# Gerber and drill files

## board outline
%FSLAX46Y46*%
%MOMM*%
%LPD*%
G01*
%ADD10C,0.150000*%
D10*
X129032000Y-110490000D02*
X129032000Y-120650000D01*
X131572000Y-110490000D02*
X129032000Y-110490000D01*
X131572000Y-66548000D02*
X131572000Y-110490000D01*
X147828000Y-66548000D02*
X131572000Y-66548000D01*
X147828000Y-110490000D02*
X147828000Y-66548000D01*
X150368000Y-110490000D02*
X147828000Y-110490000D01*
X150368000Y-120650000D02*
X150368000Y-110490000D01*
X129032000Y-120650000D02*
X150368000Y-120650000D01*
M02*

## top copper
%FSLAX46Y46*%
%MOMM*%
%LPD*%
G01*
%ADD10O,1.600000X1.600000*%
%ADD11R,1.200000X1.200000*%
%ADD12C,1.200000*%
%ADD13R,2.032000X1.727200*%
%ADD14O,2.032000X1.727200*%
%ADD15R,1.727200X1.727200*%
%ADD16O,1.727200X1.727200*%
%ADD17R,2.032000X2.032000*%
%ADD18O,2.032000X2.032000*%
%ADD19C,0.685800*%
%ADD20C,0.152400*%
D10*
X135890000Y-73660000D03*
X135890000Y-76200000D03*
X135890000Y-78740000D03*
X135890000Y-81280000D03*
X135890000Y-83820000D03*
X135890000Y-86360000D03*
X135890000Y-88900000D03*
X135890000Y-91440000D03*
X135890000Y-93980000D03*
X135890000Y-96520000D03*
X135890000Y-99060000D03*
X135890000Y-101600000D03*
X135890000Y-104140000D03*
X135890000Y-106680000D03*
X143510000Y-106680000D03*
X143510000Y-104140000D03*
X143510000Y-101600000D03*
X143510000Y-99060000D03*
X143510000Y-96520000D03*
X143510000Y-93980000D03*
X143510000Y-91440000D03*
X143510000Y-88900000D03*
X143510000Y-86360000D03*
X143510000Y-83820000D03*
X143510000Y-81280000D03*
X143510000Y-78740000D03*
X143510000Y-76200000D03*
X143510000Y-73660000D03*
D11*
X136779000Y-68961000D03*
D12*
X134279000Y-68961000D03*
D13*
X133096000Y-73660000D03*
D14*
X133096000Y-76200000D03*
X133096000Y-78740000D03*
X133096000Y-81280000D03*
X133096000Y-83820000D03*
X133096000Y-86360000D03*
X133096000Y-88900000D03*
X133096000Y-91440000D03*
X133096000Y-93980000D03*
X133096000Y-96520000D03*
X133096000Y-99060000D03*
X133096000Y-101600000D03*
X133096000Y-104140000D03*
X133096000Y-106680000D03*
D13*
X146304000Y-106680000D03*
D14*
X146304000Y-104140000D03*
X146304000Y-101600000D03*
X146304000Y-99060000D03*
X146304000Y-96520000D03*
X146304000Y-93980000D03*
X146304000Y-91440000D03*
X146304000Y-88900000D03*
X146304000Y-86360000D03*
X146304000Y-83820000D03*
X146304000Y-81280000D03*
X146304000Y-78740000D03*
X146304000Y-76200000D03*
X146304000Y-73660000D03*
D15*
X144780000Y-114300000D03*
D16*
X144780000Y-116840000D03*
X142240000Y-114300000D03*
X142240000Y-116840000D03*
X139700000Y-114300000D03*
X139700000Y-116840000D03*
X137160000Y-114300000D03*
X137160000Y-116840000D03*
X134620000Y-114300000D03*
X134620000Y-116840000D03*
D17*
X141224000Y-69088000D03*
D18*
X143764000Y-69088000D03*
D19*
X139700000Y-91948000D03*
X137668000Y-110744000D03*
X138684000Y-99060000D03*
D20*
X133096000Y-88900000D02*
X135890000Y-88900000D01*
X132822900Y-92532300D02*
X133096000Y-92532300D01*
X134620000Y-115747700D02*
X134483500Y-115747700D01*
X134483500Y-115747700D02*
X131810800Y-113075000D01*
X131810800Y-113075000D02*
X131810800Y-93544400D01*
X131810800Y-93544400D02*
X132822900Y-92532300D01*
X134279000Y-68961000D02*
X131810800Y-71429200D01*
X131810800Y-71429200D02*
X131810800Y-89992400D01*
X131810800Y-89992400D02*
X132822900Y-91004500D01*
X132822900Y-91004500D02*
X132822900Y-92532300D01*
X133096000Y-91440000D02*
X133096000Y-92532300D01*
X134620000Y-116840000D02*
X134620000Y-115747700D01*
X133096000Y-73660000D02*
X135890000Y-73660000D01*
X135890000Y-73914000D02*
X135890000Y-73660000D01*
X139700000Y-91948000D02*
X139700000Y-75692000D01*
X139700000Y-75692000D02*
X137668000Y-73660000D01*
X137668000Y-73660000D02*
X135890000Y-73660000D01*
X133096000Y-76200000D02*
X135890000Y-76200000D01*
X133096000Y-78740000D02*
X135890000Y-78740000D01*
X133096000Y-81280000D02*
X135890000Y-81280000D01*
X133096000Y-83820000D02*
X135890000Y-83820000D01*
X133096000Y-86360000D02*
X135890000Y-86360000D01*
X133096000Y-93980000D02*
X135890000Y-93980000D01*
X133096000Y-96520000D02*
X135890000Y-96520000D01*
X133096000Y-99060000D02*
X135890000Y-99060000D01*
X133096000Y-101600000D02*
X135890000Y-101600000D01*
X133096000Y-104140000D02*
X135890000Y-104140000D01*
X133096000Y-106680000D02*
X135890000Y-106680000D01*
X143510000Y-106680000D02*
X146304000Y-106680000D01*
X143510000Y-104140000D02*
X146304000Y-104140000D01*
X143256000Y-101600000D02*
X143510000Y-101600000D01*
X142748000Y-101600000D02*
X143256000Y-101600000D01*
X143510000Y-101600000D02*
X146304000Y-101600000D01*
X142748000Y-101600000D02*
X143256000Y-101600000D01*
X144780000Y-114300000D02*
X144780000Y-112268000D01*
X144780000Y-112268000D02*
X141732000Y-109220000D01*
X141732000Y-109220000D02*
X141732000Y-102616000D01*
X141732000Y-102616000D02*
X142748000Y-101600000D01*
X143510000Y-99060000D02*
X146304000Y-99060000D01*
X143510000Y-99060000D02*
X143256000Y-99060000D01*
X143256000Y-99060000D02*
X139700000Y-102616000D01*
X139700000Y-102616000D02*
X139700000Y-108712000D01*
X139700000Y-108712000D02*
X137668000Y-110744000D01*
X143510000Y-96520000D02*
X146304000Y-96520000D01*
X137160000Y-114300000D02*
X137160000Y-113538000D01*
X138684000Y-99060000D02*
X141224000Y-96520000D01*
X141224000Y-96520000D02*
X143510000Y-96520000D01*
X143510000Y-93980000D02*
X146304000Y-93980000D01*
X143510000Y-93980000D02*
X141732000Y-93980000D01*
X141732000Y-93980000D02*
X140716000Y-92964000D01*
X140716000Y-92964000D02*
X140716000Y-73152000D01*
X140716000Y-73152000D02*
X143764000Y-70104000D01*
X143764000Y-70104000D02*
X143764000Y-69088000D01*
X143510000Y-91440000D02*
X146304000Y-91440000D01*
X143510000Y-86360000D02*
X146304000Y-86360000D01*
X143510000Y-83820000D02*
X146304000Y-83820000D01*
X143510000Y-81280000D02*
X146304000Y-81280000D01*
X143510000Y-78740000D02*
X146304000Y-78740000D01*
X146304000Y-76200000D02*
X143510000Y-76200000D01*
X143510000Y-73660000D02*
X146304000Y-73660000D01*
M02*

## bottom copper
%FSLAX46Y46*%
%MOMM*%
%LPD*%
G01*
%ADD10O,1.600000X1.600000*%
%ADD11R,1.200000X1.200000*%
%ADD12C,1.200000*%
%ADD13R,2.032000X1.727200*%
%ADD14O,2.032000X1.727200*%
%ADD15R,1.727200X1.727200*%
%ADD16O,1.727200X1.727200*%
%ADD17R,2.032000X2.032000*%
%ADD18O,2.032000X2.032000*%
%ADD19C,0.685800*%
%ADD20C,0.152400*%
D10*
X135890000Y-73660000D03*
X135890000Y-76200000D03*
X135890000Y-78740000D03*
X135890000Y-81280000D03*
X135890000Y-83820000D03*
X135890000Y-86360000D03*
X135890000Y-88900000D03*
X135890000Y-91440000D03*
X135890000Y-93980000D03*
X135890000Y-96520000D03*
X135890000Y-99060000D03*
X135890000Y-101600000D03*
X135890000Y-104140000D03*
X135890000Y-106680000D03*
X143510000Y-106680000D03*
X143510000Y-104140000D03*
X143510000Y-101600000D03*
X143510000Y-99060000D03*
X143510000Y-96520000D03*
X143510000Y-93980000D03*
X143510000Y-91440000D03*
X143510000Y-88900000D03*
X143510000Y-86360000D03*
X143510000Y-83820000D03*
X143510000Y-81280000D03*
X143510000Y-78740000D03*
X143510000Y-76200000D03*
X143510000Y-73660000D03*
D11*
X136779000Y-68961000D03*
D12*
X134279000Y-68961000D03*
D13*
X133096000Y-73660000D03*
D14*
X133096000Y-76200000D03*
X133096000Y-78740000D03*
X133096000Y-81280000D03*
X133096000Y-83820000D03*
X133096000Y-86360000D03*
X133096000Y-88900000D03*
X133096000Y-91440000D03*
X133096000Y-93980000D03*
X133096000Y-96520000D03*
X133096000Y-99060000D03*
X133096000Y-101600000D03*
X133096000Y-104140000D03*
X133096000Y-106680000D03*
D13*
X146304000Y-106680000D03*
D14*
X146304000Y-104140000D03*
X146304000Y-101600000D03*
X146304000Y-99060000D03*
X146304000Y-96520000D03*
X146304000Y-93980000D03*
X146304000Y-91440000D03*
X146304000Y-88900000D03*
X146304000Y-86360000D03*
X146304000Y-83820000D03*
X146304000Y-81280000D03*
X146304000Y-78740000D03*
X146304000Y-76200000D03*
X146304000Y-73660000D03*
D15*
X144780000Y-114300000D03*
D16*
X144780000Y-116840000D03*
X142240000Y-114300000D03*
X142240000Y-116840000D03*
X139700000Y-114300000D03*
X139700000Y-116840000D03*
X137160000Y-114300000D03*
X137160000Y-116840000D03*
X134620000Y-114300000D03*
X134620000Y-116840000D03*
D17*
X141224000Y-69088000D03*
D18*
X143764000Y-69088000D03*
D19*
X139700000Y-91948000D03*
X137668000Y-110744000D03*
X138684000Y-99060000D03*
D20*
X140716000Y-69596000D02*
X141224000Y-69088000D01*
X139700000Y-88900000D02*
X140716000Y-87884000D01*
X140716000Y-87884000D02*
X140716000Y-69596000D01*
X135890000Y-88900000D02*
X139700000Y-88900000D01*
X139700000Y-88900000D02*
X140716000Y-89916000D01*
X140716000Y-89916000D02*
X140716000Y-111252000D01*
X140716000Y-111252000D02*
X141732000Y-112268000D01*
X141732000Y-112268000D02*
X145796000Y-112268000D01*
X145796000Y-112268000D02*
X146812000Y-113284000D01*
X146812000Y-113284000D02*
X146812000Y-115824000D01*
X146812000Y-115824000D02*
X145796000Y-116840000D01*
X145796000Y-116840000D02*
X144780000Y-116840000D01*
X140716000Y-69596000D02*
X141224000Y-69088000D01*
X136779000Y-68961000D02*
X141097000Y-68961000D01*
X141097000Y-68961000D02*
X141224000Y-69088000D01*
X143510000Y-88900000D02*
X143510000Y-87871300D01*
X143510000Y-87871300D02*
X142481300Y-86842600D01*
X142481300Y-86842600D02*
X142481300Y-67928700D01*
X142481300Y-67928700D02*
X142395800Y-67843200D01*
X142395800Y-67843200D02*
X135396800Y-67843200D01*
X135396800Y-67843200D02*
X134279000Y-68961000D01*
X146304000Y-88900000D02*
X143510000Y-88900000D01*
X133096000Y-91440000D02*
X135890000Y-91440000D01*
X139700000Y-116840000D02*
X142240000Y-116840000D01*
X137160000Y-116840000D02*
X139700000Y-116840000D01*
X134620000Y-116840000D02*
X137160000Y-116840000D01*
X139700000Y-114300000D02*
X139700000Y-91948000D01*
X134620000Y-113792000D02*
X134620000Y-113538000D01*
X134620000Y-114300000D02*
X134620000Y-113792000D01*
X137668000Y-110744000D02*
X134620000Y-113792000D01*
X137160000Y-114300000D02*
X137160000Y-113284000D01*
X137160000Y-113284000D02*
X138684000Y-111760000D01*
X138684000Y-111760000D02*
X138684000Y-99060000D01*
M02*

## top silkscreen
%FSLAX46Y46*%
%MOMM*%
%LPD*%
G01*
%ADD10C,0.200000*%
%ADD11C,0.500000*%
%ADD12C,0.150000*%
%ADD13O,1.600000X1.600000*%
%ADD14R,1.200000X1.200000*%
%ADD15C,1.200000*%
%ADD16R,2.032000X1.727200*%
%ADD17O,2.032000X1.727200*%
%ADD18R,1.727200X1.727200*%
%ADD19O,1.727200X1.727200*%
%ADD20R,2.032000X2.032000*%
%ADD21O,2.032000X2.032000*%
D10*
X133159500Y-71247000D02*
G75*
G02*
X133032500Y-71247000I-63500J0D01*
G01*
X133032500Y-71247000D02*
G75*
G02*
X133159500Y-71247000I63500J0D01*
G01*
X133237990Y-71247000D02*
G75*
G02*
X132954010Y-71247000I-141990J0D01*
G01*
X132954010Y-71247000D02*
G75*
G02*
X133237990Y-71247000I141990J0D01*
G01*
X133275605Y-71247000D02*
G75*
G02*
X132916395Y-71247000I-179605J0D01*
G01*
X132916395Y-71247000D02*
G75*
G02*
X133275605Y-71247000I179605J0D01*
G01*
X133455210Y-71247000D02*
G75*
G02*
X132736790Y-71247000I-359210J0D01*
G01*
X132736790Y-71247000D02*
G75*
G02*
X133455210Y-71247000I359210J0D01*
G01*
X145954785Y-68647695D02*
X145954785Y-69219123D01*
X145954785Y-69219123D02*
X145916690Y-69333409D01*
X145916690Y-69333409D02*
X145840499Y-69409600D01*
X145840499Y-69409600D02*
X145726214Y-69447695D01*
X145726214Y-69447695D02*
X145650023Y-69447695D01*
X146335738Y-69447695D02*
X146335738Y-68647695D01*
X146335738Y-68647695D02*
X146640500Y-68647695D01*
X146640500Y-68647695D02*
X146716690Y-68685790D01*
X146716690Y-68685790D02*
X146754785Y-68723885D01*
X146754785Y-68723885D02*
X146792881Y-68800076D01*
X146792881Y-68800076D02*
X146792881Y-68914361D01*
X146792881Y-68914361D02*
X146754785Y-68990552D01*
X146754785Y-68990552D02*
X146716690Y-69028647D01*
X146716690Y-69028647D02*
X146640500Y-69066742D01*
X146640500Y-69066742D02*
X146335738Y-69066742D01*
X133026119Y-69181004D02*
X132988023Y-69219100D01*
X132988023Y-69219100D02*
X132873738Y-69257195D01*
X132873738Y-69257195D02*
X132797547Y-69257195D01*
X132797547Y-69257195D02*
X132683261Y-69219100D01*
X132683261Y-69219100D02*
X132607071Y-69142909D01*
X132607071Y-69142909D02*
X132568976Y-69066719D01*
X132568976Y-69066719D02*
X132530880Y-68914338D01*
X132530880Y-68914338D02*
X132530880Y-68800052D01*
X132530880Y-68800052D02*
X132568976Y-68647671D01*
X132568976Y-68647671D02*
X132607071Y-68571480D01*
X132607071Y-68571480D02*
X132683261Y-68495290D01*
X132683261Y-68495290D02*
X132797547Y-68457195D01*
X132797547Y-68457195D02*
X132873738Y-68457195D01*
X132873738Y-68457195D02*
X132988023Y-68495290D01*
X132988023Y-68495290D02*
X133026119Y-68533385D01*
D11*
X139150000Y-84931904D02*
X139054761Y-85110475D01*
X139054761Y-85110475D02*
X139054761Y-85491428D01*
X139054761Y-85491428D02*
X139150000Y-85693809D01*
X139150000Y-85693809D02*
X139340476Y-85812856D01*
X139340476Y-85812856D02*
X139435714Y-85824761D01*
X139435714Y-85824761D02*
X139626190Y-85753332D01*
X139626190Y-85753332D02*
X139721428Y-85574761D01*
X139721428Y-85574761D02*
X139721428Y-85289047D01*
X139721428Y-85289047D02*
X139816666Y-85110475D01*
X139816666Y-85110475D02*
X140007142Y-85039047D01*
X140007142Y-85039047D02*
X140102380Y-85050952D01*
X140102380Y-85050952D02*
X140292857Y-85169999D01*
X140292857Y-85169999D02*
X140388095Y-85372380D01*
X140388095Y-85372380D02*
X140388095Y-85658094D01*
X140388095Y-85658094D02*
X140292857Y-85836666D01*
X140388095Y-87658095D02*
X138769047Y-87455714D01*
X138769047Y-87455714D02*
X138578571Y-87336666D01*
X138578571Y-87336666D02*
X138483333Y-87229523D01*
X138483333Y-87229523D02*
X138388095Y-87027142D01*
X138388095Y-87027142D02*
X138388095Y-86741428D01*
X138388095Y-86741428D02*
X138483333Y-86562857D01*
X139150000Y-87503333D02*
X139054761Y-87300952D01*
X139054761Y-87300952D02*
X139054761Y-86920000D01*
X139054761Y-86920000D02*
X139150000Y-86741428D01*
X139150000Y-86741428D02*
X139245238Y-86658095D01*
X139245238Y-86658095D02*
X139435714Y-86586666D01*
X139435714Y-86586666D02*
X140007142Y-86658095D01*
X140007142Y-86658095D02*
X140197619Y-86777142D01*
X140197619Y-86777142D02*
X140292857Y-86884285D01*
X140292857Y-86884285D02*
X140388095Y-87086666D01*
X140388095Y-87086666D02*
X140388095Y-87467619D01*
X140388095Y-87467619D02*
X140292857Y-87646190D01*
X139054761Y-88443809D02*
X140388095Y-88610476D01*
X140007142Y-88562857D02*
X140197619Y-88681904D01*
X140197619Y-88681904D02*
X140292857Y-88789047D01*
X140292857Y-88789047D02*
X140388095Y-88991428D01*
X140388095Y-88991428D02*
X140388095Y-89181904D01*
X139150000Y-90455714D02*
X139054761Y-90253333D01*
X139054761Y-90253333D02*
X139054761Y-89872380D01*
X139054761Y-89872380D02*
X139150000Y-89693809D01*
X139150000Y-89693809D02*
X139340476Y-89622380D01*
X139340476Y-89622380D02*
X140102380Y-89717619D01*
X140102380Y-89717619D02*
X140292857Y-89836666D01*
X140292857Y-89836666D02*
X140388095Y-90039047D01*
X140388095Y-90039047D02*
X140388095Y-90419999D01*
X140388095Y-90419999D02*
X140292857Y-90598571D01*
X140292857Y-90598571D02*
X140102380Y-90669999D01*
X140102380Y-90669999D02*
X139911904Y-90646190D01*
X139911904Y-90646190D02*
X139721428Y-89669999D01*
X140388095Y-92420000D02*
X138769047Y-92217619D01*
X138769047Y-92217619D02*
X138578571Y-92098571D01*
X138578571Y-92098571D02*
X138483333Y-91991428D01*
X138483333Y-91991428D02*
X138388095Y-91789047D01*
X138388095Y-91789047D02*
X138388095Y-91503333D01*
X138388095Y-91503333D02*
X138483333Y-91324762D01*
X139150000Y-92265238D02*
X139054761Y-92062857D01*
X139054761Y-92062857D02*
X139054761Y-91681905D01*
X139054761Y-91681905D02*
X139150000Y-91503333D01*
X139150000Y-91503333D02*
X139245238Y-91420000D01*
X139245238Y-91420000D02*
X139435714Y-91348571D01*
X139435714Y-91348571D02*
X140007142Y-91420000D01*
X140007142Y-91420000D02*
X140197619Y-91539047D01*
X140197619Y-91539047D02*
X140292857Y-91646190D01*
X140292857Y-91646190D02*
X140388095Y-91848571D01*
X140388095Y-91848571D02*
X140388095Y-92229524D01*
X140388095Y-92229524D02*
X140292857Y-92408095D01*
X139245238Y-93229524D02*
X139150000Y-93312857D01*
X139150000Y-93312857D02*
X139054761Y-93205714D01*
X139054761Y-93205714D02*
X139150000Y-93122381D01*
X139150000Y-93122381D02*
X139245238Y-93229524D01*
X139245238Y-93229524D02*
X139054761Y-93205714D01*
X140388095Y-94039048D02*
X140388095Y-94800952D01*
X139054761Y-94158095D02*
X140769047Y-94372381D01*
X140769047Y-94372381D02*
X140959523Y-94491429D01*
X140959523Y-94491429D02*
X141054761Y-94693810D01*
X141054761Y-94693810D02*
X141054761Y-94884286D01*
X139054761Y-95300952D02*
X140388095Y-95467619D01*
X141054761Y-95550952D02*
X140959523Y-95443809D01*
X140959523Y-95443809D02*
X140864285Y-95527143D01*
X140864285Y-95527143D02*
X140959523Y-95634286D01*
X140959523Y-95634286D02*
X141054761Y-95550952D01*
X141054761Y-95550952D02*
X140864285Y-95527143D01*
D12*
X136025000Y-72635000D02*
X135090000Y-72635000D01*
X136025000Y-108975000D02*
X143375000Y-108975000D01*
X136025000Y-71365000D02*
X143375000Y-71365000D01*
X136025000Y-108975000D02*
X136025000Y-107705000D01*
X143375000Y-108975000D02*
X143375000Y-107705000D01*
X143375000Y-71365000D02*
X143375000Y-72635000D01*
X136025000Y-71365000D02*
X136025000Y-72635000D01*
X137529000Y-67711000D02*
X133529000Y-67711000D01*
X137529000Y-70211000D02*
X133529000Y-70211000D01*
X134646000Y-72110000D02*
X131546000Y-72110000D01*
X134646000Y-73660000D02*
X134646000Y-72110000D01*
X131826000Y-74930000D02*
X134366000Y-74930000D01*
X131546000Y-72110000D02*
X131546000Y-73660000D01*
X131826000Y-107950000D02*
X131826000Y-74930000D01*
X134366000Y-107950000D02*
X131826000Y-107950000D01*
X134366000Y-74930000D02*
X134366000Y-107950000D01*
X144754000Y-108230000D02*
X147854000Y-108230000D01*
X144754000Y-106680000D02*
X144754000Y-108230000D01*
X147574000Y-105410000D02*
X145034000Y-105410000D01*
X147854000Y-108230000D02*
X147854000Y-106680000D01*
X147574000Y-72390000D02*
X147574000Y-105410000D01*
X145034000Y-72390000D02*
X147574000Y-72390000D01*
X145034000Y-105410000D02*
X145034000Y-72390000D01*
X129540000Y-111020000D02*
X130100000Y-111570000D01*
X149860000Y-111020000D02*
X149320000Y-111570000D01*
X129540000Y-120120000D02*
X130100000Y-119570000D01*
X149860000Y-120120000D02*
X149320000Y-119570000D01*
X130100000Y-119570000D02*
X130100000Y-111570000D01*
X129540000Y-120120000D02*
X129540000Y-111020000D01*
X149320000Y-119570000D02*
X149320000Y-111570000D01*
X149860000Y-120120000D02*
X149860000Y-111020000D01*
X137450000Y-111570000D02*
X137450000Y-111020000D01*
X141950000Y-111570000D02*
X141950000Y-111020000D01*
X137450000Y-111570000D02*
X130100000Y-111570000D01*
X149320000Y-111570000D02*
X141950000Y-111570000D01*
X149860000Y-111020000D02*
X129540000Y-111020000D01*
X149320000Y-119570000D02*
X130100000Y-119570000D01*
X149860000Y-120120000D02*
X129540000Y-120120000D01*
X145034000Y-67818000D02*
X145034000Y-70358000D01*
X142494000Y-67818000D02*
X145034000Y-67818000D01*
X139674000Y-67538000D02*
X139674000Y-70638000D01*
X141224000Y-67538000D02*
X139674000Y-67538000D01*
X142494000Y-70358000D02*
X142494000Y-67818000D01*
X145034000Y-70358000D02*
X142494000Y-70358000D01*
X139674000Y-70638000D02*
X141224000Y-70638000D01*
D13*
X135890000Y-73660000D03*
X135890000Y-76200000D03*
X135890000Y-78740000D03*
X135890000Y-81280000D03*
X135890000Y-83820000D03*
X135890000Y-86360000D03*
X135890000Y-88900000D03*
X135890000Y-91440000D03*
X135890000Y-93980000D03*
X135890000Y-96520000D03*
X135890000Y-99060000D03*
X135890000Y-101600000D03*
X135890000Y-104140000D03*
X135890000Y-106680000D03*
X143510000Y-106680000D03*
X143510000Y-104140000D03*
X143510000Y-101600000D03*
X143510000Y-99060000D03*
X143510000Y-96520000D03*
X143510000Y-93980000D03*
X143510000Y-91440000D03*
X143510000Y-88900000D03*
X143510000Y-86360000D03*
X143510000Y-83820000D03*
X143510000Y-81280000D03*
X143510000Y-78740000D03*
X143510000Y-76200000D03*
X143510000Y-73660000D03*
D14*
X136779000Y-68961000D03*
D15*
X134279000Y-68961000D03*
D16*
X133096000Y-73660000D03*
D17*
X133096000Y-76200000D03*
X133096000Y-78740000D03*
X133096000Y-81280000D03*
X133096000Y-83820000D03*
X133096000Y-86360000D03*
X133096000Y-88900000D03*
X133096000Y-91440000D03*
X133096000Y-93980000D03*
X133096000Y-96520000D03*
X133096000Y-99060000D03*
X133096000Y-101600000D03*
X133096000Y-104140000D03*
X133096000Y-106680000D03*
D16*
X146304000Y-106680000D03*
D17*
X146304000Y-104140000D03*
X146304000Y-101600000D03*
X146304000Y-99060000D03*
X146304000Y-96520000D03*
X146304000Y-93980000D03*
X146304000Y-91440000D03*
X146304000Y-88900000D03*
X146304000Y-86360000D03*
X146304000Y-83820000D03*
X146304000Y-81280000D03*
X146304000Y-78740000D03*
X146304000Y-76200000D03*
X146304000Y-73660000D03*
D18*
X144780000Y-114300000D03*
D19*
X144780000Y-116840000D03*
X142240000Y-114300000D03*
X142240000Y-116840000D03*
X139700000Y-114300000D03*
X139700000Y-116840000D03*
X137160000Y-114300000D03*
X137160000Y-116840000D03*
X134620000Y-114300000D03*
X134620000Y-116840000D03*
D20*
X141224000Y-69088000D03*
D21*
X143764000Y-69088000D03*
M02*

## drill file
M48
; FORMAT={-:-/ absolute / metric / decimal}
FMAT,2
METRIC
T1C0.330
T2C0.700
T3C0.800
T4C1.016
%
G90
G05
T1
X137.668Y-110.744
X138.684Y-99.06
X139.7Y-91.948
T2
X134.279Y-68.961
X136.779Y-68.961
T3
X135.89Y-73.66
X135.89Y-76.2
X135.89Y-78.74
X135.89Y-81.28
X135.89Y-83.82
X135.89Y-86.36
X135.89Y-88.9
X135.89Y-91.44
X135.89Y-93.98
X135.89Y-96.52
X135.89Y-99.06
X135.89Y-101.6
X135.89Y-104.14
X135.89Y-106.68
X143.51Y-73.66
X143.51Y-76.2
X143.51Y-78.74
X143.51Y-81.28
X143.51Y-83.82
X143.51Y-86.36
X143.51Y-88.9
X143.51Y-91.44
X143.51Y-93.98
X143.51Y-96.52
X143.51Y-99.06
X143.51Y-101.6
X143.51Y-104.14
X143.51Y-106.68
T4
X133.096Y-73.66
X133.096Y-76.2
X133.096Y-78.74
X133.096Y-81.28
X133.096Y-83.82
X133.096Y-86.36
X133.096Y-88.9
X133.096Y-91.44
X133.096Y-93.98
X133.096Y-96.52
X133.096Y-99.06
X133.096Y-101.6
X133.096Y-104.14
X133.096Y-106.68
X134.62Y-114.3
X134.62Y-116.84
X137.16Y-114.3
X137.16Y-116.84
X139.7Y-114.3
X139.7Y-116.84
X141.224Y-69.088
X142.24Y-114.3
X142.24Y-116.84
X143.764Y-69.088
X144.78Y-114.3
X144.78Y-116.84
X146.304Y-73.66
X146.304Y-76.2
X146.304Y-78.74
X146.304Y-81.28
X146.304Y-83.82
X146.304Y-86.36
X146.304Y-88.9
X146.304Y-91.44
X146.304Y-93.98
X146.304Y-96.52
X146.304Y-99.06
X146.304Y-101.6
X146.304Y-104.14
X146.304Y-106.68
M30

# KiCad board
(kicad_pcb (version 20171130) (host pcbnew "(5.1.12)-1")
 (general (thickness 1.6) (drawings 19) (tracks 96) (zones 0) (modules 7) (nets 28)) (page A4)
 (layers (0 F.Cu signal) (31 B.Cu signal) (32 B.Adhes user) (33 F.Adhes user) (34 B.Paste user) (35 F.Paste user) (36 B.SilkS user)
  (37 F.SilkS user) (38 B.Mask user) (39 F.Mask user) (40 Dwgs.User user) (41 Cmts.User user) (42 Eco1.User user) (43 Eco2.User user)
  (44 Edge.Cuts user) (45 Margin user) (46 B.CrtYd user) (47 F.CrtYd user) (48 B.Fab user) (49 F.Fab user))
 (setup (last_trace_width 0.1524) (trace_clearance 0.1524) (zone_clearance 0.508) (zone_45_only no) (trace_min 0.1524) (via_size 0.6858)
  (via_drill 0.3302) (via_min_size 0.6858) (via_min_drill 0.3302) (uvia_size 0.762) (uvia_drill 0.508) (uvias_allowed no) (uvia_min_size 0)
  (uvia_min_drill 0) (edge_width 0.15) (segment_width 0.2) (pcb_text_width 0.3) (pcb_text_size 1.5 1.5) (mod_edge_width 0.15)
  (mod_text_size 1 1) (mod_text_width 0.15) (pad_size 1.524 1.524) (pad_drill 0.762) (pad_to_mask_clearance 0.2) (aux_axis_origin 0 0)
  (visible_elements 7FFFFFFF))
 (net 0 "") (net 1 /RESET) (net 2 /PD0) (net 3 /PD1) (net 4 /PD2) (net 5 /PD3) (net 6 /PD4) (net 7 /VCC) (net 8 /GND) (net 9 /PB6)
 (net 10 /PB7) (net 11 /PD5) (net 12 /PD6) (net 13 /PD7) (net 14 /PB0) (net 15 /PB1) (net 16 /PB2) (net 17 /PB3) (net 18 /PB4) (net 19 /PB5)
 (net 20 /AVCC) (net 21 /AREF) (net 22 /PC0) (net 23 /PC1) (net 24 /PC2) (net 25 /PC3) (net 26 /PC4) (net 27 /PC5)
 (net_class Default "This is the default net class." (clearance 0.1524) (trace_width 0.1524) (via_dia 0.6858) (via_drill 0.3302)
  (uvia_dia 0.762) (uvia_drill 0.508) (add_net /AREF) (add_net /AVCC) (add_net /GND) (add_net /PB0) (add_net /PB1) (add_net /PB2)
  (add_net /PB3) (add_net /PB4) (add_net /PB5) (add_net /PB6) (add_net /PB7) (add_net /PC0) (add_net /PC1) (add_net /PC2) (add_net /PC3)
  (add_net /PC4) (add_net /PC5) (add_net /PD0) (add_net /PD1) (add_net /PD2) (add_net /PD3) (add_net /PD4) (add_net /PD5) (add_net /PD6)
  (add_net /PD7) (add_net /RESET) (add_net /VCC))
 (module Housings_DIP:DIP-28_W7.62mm (layer F.Cu) (at 135.89 73.66)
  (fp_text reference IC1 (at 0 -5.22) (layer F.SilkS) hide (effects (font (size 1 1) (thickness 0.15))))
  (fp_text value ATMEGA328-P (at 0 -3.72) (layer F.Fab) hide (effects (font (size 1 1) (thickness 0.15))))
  (fp_line (start 0.135 -1.025) (end -0.8 -1.025) (layer F.SilkS) (width 0.15))
  (fp_line (start 0.135 35.315) (end 7.485 35.315) (layer F.SilkS) (width 0.15))
  (fp_line (start 0.135 -2.295) (end 7.485 -2.295) (layer F.SilkS) (width 0.15))
  (fp_line (start 0.135 35.315) (end 0.135 34.045) (layer F.SilkS) (width 0.15))
  (fp_line (start 7.485 35.315) (end 7.485 34.045) (layer F.SilkS) (width 0.15))
  (fp_line (start 7.485 -2.295) (end 7.485 -1.025) (layer F.SilkS) (width 0.15))
  (fp_line (start 0.135 -2.295) (end 0.135 -1.025) (layer F.SilkS) (width 0.15))
  (pad 1 thru_hole oval (at 0 0) (size 1.6 1.6) (drill 0.8) (layers *.Cu *.Mask F.SilkS) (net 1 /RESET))
  (pad 2 thru_hole oval (at 0 2.54) (size 1.6 1.6) (drill 0.8) (layers *.Cu *.Mask F.SilkS) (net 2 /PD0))
  (pad 3 thru_hole oval (at 0 5.08) (size 1.6 1.6) (drill 0.8) (layers *.Cu *.Mask F.SilkS) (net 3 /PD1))
  (pad 4 thru_hole oval (at 0 7.62) (size 1.6 1.6) (drill 0.8) (layers *.Cu *.Mask F.SilkS) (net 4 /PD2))
  (pad 5 thru_hole oval (at 0 10.16) (size 1.6 1.6) (drill 0.8) (layers *.Cu *.Mask F.SilkS) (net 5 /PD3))
  (pad 6 thru_hole oval (at 0 12.7) (size 1.6 1.6) (drill 0.8) (layers *.Cu *.Mask F.SilkS) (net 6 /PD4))
  (pad 7 thru_hole oval (at 0 15.24) (size 1.6 1.6) (drill 0.8) (layers *.Cu *.Mask F.SilkS) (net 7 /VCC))
  (pad 8 thru_hole oval (at 0 17.78) (size 1.6 1.6) (drill 0.8) (layers *.Cu *.Mask F.SilkS) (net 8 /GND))
  (pad 9 thru_hole oval (at 0 20.32) (size 1.6 1.6) (drill 0.8) (layers *.Cu *.Mask F.SilkS) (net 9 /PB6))
  (pad 10 thru_hole oval (at 0 22.86) (size 1.6 1.6) (drill 0.8) (layers *.Cu *.Mask F.SilkS) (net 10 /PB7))
  (pad 11 thru_hole oval (at 0 25.4) (size 1.6 1.6) (drill 0.8) (layers *.Cu *.Mask F.SilkS) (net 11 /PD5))
  (pad 12 thru_hole oval (at 0 27.94) (size 1.6 1.6) (drill 0.8) (layers *.Cu *.Mask F.SilkS) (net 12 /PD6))
  (pad 13 thru_hole oval (at 0 30.48) (size 1.6 1.6) (drill 0.8) (layers *.Cu *.Mask F.SilkS) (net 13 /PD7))
  (pad 14 thru_hole oval (at 0 33.02) (size 1.6 1.6) (drill 0.8) (layers *.Cu *.Mask F.SilkS) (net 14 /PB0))
  (pad 15 thru_hole oval (at 7.62 33.02) (size 1.6 1.6) (drill 0.8) (layers *.Cu *.Mask F.SilkS) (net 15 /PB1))
  (pad 16 thru_hole oval (at 7.62 30.48) (size 1.6 1.6) (drill 0.8) (layers *.Cu *.Mask F.SilkS) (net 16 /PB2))
  (pad 17 thru_hole oval (at 7.62 27.94) (size 1.6 1.6) (drill 0.8) (layers *.Cu *.Mask F.SilkS) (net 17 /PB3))
  (pad 18 thru_hole oval (at 7.62 25.4) (size 1.6 1.6) (drill 0.8) (layers *.Cu *.Mask F.SilkS) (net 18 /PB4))
  (pad 19 thru_hole oval (at 7.62 22.86) (size 1.6 1.6) (drill 0.8) (layers *.Cu *.Mask F.SilkS) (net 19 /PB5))
  (pad 20 thru_hole oval (at 7.62 20.32) (size 1.6 1.6) (drill 0.8) (layers *.Cu *.Mask F.SilkS) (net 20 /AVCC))
  (pad 21 thru_hole oval (at 7.62 17.78) (size 1.6 1.6) (drill 0.8) (layers *.Cu *.Mask F.SilkS) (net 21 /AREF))
  (pad 22 thru_hole oval (at 7.62 15.24) (size 1.6 1.6) (drill 0.8) (layers *.Cu *.Mask F.SilkS) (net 8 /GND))
  (pad 23 thru_hole oval (at 7.62 12.7) (size 1.6 1.6) (drill 0.8) (layers *.Cu *.Mask F.SilkS) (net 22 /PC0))
  (pad 24 thru_hole oval (at 7.62 10.16) (size 1.6 1.6) (drill 0.8) (layers *.Cu *.Mask F.SilkS) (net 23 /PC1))
  (pad 25 thru_hole oval (at 7.62 7.62) (size 1.6 1.6) (drill 0.8) (layers *.Cu *.Mask F.SilkS) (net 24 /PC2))
  (pad 26 thru_hole oval (at 7.62 5.08) (size 1.6 1.6) (drill 0.8) (layers *.Cu *.Mask F.SilkS) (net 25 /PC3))
  (pad 27 thru_hole oval (at 7.62 2.54) (size 1.6 1.6) (drill 0.8) (layers *.Cu *.Mask F.SilkS) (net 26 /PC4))
  (pad 28 thru_hole oval (at 7.62 0) (size 1.6 1.6) (drill 0.8) (layers *.Cu *.Mask F.SilkS) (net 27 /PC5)))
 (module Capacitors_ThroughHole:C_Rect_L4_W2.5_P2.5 (layer F.Cu) (at 136.779 68.961 180)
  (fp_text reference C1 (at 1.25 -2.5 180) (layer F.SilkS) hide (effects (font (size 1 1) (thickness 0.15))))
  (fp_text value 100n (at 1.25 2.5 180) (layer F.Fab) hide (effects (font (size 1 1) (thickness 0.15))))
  (fp_line (start -0.75 1.25) (end 3.25 1.25) (layer F.SilkS) (width 0.15))
  (fp_line (start -0.75 -1.25) (end 3.25 -1.25) (layer F.SilkS) (width 0.15))
  (pad 1 thru_hole rect (at 0 0 180) (size 1.2 1.2) (drill 0.7) (layers *.Cu *.Mask F.SilkS) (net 7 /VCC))
  (pad 2 thru_hole circle (at 2.5 0 180) (size 1.2 1.2) (drill 0.7) (layers *.Cu *.Mask F.SilkS) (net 8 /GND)))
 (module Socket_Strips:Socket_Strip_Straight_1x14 (layer F.Cu) (at 133.096 73.66 270)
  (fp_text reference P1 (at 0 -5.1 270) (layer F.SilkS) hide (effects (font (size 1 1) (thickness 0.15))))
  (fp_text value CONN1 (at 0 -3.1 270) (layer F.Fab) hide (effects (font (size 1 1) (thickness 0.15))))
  (fp_line (start -1.55 -1.55) (end -1.55 1.55) (layer F.SilkS) (width 0.15))
  (fp_line (start 0 -1.55) (end -1.55 -1.55) (layer F.SilkS) (width 0.15))
  (fp_line (start 1.27 1.27) (end 1.27 -1.27) (layer F.SilkS) (width 0.15))
  (fp_line (start -1.55 1.55) (end 0 1.55) (layer F.SilkS) (width 0.15))
  (fp_line (start 34.29 1.27) (end 1.27 1.27) (layer F.SilkS) (width 0.15))
  (fp_line (start 34.29 -1.27) (end 34.29 1.27) (layer F.SilkS) (width 0.15))
  (fp_line (start 1.27 -1.27) (end 34.29 -1.27) (layer F.SilkS) (width 0.15))
  (pad 1 thru_hole rect (at 0 0 270) (size 1.7272 2.032) (drill 1.016) (layers *.Cu *.Mask F.SilkS) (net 1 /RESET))
  (pad 2 thru_hole oval (at 2.54 0 270) (size 1.7272 2.032) (drill 1.016) (layers *.Cu *.Mask F.SilkS) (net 2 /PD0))
  (pad 3 thru_hole oval (at 5.08 0 270) (size 1.7272 2.032) (drill 1.016) (layers *.Cu *.Mask F.SilkS) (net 3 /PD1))
  (pad 4 thru_hole oval (at 7.62 0 270) (size 1.7272 2.032) (drill 1.016) (layers *.Cu *.Mask F.SilkS) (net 4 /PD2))
  (pad 5 thru_hole oval (at 10.16 0 270) (size 1.7272 2.032) (drill 1.016) (layers *.Cu *.Mask F.SilkS) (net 5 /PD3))
  (pad 6 thru_hole oval (at 12.7 0 270) (size 1.7272 2.032) (drill 1.016) (layers *.Cu *.Mask F.SilkS) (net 6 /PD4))
  (pad 7 thru_hole oval (at 15.24 0 270) (size 1.7272 2.032) (drill 1.016) (layers *.Cu *.Mask F.SilkS) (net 7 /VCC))
  (pad 8 thru_hole oval (at 17.78 0 270) (size 1.7272 2.032) (drill 1.016) (layers *.Cu *.Mask F.SilkS) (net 8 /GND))
  (pad 9 thru_hole oval (at 20.32 0 270) (size 1.7272 2.032) (drill 1.016) (layers *.Cu *.Mask F.SilkS) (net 9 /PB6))
  (pad 10 thru_hole oval (at 22.86 0 270) (size 1.7272 2.032) (drill 1.016) (layers *.Cu *.Mask F.SilkS) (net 10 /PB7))
  (pad 11 thru_hole oval (at 25.4 0 270) (size 1.7272 2.032) (drill 1.016) (layers *.Cu *.Mask F.SilkS) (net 11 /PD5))
  (pad 12 thru_hole oval (at 27.94 0 270) (size 1.7272 2.032) (drill 1.016) (layers *.Cu *.Mask F.SilkS) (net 12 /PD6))
  (pad 13 thru_hole oval (at 30.48 0 270) (size 1.7272 2.032) (drill 1.016) (layers *.Cu *.Mask F.SilkS) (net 13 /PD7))
  (pad 14 thru_hole oval (at 33.02 0 270) (size 1.7272 2.032) (drill 1.016) (layers *.Cu *.Mask F.SilkS) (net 14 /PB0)))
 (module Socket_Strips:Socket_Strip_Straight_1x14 (layer F.Cu) (at 146.304 106.68 90)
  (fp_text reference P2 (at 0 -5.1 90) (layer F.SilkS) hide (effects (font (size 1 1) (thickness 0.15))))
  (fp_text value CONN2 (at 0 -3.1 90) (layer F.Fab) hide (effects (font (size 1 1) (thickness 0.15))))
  (fp_line (start -1.55 -1.55) (end -1.55 1.55) (layer F.SilkS) (width 0.15))
  (fp_line (start 0 -1.55) (end -1.55 -1.55) (layer F.SilkS) (width 0.15))
  (fp_line (start 1.27 1.27) (end 1.27 -1.27) (layer F.SilkS) (width 0.15))
  (fp_line (start -1.55 1.55) (end 0 1.55) (layer F.SilkS) (width 0.15))
  (fp_line (start 34.29 1.27) (end 1.27 1.27) (layer F.SilkS) (width 0.15))
  (fp_line (start 34.29 -1.27) (end 34.29 1.27) (layer F.SilkS) (width 0.15))
  (fp_line (start 1.27 -1.27) (end 34.29 -1.27) (layer F.SilkS) (width 0.15))
  (pad 1 thru_hole rect (at 0 0 90) (size 1.7272 2.032) (drill 1.016) (layers *.Cu *.Mask F.SilkS) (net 15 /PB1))
  (pad 2 thru_hole oval (at 2.54 0 90) (size 1.7272 2.032) (drill 1.016) (layers *.Cu *.Mask F.SilkS) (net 16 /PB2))
  (pad 3 thru_hole oval (at 5.08 0 90) (size 1.7272 2.032) (drill 1.016) (layers *.Cu *.Mask F.SilkS) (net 17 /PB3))
  (pad 4 thru_hole oval (at 7.62 0 90) (size 1.7272 2.032) (drill 1.016) (layers *.Cu *.Mask F.SilkS) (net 18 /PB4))
  (pad 5 thru_hole oval (at 10.16 0 90) (size 1.7272 2.032) (drill 1.016) (layers *.Cu *.Mask F.SilkS) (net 19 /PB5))
  (pad 6 thru_hole oval (at 12.7 0 90) (size 1.7272 2.032) (drill 1.016) (layers *.Cu *.Mask F.SilkS) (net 20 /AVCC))
  (pad 7 thru_hole oval (at 15.24 0 90) (size 1.7272 2.032) (drill 1.016) (layers *.Cu *.Mask F.SilkS) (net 21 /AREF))
  (pad 8 thru_hole oval (at 17.78 0 90) (size 1.7272 2.032) (drill 1.016) (layers *.Cu *.Mask F.SilkS) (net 8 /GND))
  (pad 9 thru_hole oval (at 20.32 0 90) (size 1.7272 2.032) (drill 1.016) (layers *.Cu *.Mask F.SilkS) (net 22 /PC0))
  (pad 10 thru_hole oval (at 22.86 0 90) (size 1.7272 2.032) (drill 1.016) (layers *.Cu *.Mask F.SilkS) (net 23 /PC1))
  (pad 11 thru_hole oval (at 25.4 0 90) (size 1.7272 2.032) (drill 1.016) (layers *.Cu *.Mask F.SilkS) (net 24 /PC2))
  (pad 12 thru_hole oval (at 27.94 0 90) (size 1.7272 2.032) (drill 1.016) (layers *.Cu *.Mask F.SilkS) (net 25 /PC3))
  (pad 13 thru_hole oval (at 30.48 0 90) (size 1.7272 2.032) (drill 1.016) (layers *.Cu *.Mask F.SilkS) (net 26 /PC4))
  (pad 14 thru_hole oval (at 33.02 0 90) (size 1.7272 2.032) (drill 1.016) (layers *.Cu *.Mask F.SilkS) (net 27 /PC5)))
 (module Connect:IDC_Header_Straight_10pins (layer F.Cu) (at 144.78 114.3 180)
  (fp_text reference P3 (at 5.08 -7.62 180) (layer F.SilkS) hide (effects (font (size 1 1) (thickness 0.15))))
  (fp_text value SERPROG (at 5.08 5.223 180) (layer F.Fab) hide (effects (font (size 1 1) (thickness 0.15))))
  (fp_line (start 15.24 3.28) (end 14.68 2.73) (layer F.SilkS) (width 0.15))
  (fp_line (start -5.08 3.28) (end -4.54 2.73) (layer F.SilkS) (width 0.15))
  (fp_line (start 15.24 -5.82) (end 14.68 -5.27) (layer F.SilkS) (width 0.15))
  (fp_line (start -5.08 -5.82) (end -4.54 -5.27) (layer F.SilkS) (width 0.15))
  (fp_line (start 14.68 -5.27) (end 14.68 2.73) (layer F.SilkS) (width 0.15))
  (fp_line (start 15.24 -5.82) (end 15.24 3.28) (layer F.SilkS) (width 0.15))
  (fp_line (start -4.54 -5.27) (end -4.54 2.73) (layer F.SilkS) (width 0.15))
  (fp_line (start -5.08 -5.82) (end -5.08 3.28) (layer F.SilkS) (width 0.15))
  (fp_line (start 7.33 2.73) (end 7.33 3.28) (layer F.SilkS) (width 0.15))
  (fp_line (start 2.83 2.73) (end 2.83 3.28) (layer F.SilkS) (width 0.15))
  (fp_line (start 7.33 2.73) (end 14.68 2.73) (layer F.SilkS) (width 0.15))
  (fp_line (start -4.54 2.73) (end 2.83 2.73) (layer F.SilkS) (width 0.15))
  (fp_line (start -5.08 3.28) (end 15.24 3.28) (layer F.SilkS) (width 0.15))
  (fp_line (start -4.54 -5.27) (end 14.68 -5.27) (layer F.SilkS) (width 0.15))
  (fp_line (start -5.08 -5.82) (end 15.24 -5.82) (layer F.SilkS) (width 0.15))
  (pad 1 thru_hole rect (at 0 0 180) (size 1.7272 1.7272) (drill 1.016) (layers *.Cu *.Mask F.SilkS) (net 17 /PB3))
  (pad 2 thru_hole oval (at 0 -2.54 180) (size 1.7272 1.7272) (drill 1.016) (layers *.Cu *.Mask F.SilkS) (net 7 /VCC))
  (pad 3 thru_hole oval (at 2.54 0 180) (size 1.7272 1.7272) (drill 1.016) (layers *.Cu *.Mask F.SilkS))
  (pad 4 thru_hole oval (at 2.54 -2.54 180) (size 1.7272 1.7272) (drill 1.016) (layers *.Cu *.Mask F.SilkS) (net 8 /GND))
  (pad 5 thru_hole oval (at 5.08 0 180) (size 1.7272 1.7272) (drill 1.016) (layers *.Cu *.Mask F.SilkS) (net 1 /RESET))
  (pad 6 thru_hole oval (at 5.08 -2.54 180) (size 1.7272 1.7272) (drill 1.016) (layers *.Cu *.Mask F.SilkS) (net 8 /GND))
  (pad 7 thru_hole oval (at 7.62 0 180) (size 1.7272 1.7272) (drill 1.016) (layers *.Cu *.Mask F.SilkS) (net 19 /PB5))
  (pad 8 thru_hole oval (at 7.62 -2.54 180) (size 1.7272 1.7272) (drill 1.016) (layers *.Cu *.Mask F.SilkS) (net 8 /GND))
  (pad 9 thru_hole oval (at 10.16 0 180) (size 1.7272 1.7272) (drill 1.016) (layers *.Cu *.Mask F.SilkS) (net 18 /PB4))
  (pad 10 thru_hole oval (at 10.16 -2.54 180) (size 1.7272 1.7272) (drill 1.016) (layers *.Cu *.Mask F.SilkS) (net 8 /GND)))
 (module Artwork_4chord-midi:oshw (layer B.Cu) (at 139.7 109.474 180)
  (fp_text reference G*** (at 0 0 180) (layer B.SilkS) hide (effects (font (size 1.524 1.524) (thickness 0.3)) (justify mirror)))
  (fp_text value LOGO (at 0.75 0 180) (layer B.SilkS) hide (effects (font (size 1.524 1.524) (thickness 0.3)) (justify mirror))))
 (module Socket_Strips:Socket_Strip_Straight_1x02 (layer F.Cu) (at 141.224 69.088)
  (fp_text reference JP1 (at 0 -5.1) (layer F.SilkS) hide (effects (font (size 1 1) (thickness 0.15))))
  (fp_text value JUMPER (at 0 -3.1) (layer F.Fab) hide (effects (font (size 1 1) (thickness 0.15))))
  (fp_line (start 3.81 -1.27) (end 3.81 1.27) (layer F.SilkS) (width 0.15))
  (fp_line (start 1.27 -1.27) (end 3.81 -1.27) (layer F.SilkS) (width 0.15))
  (fp_line (start -1.55 -1.55) (end -1.55 1.55) (layer F.SilkS) (width 0.15))
  (fp_line (start 0 -1.55) (end -1.55 -1.55) (layer F.SilkS) (width 0.15))
  (fp_line (start 1.27 1.27) (end 1.27 -1.27) (layer F.SilkS) (width 0.15))
  (fp_line (start 3.81 1.27) (end 1.27 1.27) (layer F.SilkS) (width 0.15))
  (fp_line (start -1.55 1.55) (end 0 1.55) (layer F.SilkS) (width 0.15))
  (pad 1 thru_hole rect (at 0 0) (size 2.032 2.032) (drill 1.016) (layers *.Cu *.Mask F.SilkS) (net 7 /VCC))
  (pad 2 thru_hole oval (at 2.54 0) (size 2.032 2.032) (drill 1.016) (layers *.Cu *.Mask F.SilkS) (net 20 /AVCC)))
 (gr_circle (center 133.096 71.247) (end 133.096 71.3105) (layer F.SilkS) (width 0.2))
 (gr_circle (center 133.096 71.247) (end 133.1595 71.374) (layer F.SilkS) (width 0.2))
 (gr_circle (center 133.096 71.247) (end 133.223 71.374) (layer F.SilkS) (width 0.2))
 (gr_circle (center 133.096 71.247) (end 133.35 71.501) (layer F.SilkS) (width 0.2))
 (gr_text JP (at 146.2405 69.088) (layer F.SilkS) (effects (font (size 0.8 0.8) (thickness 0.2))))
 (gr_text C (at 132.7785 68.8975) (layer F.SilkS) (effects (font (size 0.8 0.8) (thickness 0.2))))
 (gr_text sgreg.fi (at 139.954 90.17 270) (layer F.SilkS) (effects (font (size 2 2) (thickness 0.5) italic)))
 (gr_line (start 129.032 110.49) (end 129.032 120.65) (angle 90) (layer Edge.Cuts) (width 0.15))
 (gr_line (start 131.572 110.49) (end 129.032 110.49) (angle 90) (layer Edge.Cuts) (width 0.15))
 (gr_line (start 131.572 66.548) (end 131.572 110.49) (angle 90) (layer Edge.Cuts) (width 0.15))
 (gr_line (start 147.828 66.548) (end 131.572 66.548) (angle 90) (layer Edge.Cuts) (width 0.15))
 (gr_line (start 147.828 110.49) (end 147.828 66.548) (angle 90) (layer Edge.Cuts) (width 0.15))
 (gr_line (start 150.368 110.49) (end 147.828 110.49) (angle 90) (layer Edge.Cuts) (width 0.15))
 (gr_line (start 150.368 120.65) (end 150.368 110.49) (angle 90) (layer Edge.Cuts) (width 0.15))
 (gr_line (start 129.032 120.65) (end 150.368 120.65) (angle 90) (layer Edge.Cuts) (width 0.15))
 (segment (start 140.716 69.596) (end 141.224 69.088) (width 0.1524) (layer B.Cu) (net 7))
 (segment (start 139.7 88.9) (end 140.716 87.884) (width 0.1524) (layer B.Cu) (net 7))
 (segment (start 140.716 87.884) (end 140.716 69.596) (width 0.1524) (layer B.Cu) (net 7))
 (segment (start 135.89 88.9) (end 139.7 88.9) (width 0.1524) (layer B.Cu) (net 7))
 (segment (start 133.096 88.9) (end 135.89 88.9) (width 0.1524) (layer F.Cu) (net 7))
 (segment (start 139.7 88.9) (end 140.716 89.916) (width 0.1524) (layer B.Cu) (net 7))
 (segment (start 140.716 89.916) (end 140.716 111.252) (width 0.1524) (layer B.Cu) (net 7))
 (segment (start 140.716 111.252) (end 141.732 112.268) (width 0.1524) (layer B.Cu) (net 7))
 (segment (start 141.732 112.268) (end 145.796 112.268) (width 0.1524) (layer B.Cu) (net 7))
 (segment (start 145.796 112.268) (end 146.812 113.284) (width 0.1524) (layer B.Cu) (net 7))
 (segment (start 146.812 113.284) (end 146.812 115.824) (width 0.1524) (layer B.Cu) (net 7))
 (segment (start 146.812 115.824) (end 145.796 116.84) (width 0.1524) (layer B.Cu) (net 7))
 (segment (start 145.796 116.84) (end 144.78 116.84) (width 0.1524) (layer B.Cu) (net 7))
 (segment (start 140.716 69.596) (end 141.224 69.088) (width 0.1524) (layer B.Cu) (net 7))
 (segment (start 136.779 68.961) (end 141.097 68.961) (width 0.1524) (layer B.Cu) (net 7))
 (segment (start 141.097 68.961) (end 141.224 69.088) (width 0.1524) (layer B.Cu) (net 7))
 (segment (start 143.51 88.9) (end 143.51 87.8713) (width 0.1524) (layer B.Cu) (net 8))
 (segment (start 143.51 87.8713) (end 142.4813 86.8426) (width 0.1524) (layer B.Cu) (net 8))
 (segment (start 142.4813 86.8426) (end 142.4813 67.9287) (width 0.1524) (layer B.Cu) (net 8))
 (segment (start 142.4813 67.9287) (end 142.3958 67.8432) (width 0.1524) (layer B.Cu) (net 8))
 (segment (start 142.3958 67.8432) (end 135.3968 67.8432) (width 0.1524) (layer B.Cu) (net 8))
 (segment (start 135.3968 67.8432) (end 134.279 68.961) (width 0.1524) (layer B.Cu) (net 8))
 (segment (start 146.304 88.9) (end 143.51 88.9) (width 0.1524) (layer B.Cu) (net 8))
 (segment (start 132.8229 92.5323) (end 133.096 92.5323) (width 0.1524) (layer F.Cu) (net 8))
 (segment (start 134.62 115.7477) (end 134.4835 115.7477) (width 0.1524) (layer F.Cu) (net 8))
 (segment (start 134.4835 115.7477) (end 131.8108 113.075) (width 0.1524) (layer F.Cu) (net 8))
 (segment (start 131.8108 113.075) (end 131.8108 93.5444) (width 0.1524) (layer F.Cu) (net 8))
 (segment (start 131.8108 93.5444) (end 132.8229 92.5323) (width 0.1524) (layer F.Cu) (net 8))
 (segment (start 134.279 68.961) (end 131.8108 71.4292) (width 0.1524) (layer F.Cu) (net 8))
 (segment (start 131.8108 71.4292) (end 131.8108 89.9924) (width 0.1524) (layer F.Cu) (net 8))
 (segment (start 131.8108 89.9924) (end 132.8229 91.0045) (width 0.1524) (layer F.Cu) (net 8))
 (segment (start 132.8229 91.0045) (end 132.8229 92.5323) (width 0.1524) (layer F.Cu) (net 8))
 (segment (start 133.096 91.44) (end 135.89 91.44) (width 0.1524) (layer B.Cu) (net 8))
 (segment (start 133.096 91.44) (end 133.096 92.5323) (width 0.1524) (layer F.Cu) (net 8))
 (segment (start 134.62 116.84) (end 134.62 115.7477) (width 0.1524) (layer F.Cu) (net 8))
 (segment (start 139.7 116.84) (end 142.24 116.84) (width 0.1524) (layer B.Cu) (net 8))
 (segment (start 137.16 116.84) (end 139.7 116.84) (width 0.1524) (layer B.Cu) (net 8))
 (segment (start 134.62 116.84) (end 137.16 116.84) (width 0.1524) (layer B.Cu) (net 8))
 (segment (start 133.096 73.66) (end 135.89 73.66) (width 0.1524) (layer F.Cu) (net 1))
 (segment (start 135.89 73.914) (end 135.89 73.66) (width 0.1524) (layer F.Cu) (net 1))
 (segment (start 139.7 91.948) (end 139.7 75.692) (width 0.1524) (layer F.Cu) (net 1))
 (segment (start 139.7 75.692) (end 137.668 73.66) (width 0.1524) (layer F.Cu) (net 1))
 (segment (start 137.668 73.66) (end 135.89 73.66) (width 0.1524) (layer F.Cu) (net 1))
 (segment (start 139.7 114.3) (end 139.7 91.948) (width 0.1524) (layer B.Cu) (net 1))
 (via (at 139.7 91.948) (size 0.6858) (layers F.Cu B.Cu) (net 1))
 (segment (start 133.096 76.2) (end 135.89 76.2) (width 0.1524) (layer F.Cu) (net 2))
 (segment (start 133.096 78.74) (end 135.89 78.74) (width 0.1524) (layer F.Cu) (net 3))
 (segment (start 133.096 81.28) (end 135.89 81.28) (width 0.1524) (layer F.Cu) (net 4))
 (segment (start 133.096 83.82) (end 135.89 83.82) (width 0.1524) (layer F.Cu) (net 5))
 (segment (start 133.096 86.36) (end 135.89 86.36) (width 0.1524) (layer F.Cu) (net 6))
 (segment (start 133.096 93.98) (end 135.89 93.98) (width 0.1524) (layer F.Cu) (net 9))
 (segment (start 133.096 96.52) (end 135.89 96.52) (width 0.1524) (layer F.Cu) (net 10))
 (segment (start 133.096 99.06) (end 135.89 99.06) (width 0.1524) (layer F.Cu) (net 11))
 (segment (start 133.096 101.6) (end 135.89 101.6) (width 0.1524) (layer F.Cu) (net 12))
 (segment (start 133.096 104.14) (end 135.89 104.14) (width 0.1524) (layer F.Cu) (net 13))
 (segment (start 133.096 106.68) (end 135.89 106.68) (width 0.1524) (layer F.Cu) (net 14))
 (segment (start 143.51 106.68) (end 146.304 106.68) (width 0.1524) (layer F.Cu) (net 15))
 (segment (start 143.51 104.14) (end 146.304 104.14) (width 0.1524) (layer F.Cu) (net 16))
 (segment (start 143.256 101.6) (end 143.51 101.6) (width 0.1524) (layer F.Cu) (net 17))
 (segment (start 142.748 101.6) (end 143.256 101.6) (width 0.1524) (layer F.Cu) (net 17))
 (segment (start 143.51 101.6) (end 146.304 101.6) (width 0.1524) (layer F.Cu) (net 17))
 (segment (start 142.748 101.6) (end 143.256 101.6) (width 0.1524) (layer F.Cu) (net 17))
 (segment (start 144.78 114.3) (end 144.78 112.268) (width 0.1524) (layer F.Cu) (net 17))
 (segment (start 144.78 112.268) (end 141.732 109.22) (width 0.1524) (layer F.Cu) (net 17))
 (segment (start 141.732 109.22) (end 141.732 102.616) (width 0.1524) (layer F.Cu) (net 17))
 (segment (start 141.732 102.616) (end 142.748 101.6) (width 0.1524) (layer F.Cu) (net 17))
 (segment (start 134.62 113.792) (end 134.62 113.538) (width 0.1524) (layer B.Cu) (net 18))
 (segment (start 134.62 114.3) (end 134.62 113.792) (width 0.1524) (layer B.Cu) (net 18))
 (segment (start 143.51 99.06) (end 146.304 99.06) (width 0.1524) (layer F.Cu) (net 18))
 (segment (start 143.51 99.06) (end 143.256 99.06) (width 0.1524) (layer F.Cu) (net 18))
 (segment (start 143.256 99.06) (end 139.7 102.616) (width 0.1524) (layer F.Cu) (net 18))
 (segment (start 139.7 102.616) (end 139.7 108.712) (width 0.1524) (layer F.Cu) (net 18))
 (segment (start 139.7 108.712) (end 137.668 110.744) (width 0.1524) (layer F.Cu) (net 18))
 (segment (start 137.668 110.744) (end 134.62 113.792) (width 0.1524) (layer B.Cu) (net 18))
 (via (at 137.668 110.744) (size 0.6858) (layers F.Cu B.Cu) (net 18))
 (segment (start 143.51 96.52) (end 146.304 96.52) (width 0.1524) (layer F.Cu) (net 19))
 (segment (start 137.16 114.3) (end 137.16 113.538) (width 0.1524) (layer F.Cu) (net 19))
 (segment (start 137.16 114.3) (end 137.16 113.284) (width 0.1524) (layer B.Cu) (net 19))
 (segment (start 137.16 113.284) (end 138.684 111.76) (width 0.1524) (layer B.Cu) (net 19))
 (segment (start 138.684 111.76) (end 138.684 99.06) (width 0.1524) (layer B.Cu) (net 19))
 (segment (start 138.684 99.06) (end 141.224 96.52) (width 0.1524) (layer F.Cu) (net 19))
 (segment (start 141.224 96.52) (end 143.51 96.52) (width 0.1524) (layer F.Cu) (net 19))
 (via (at 138.684 99.06) (size 0.6858) (layers F.Cu B.Cu) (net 19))
 (segment (start 143.51 93.98) (end 146.304 93.98) (width 0.1524) (layer F.Cu) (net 20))
 (segment (start 143.51 93.98) (end 141.732 93.98) (width 0.1524) (layer F.Cu) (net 20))
 (segment (start 141.732 93.98) (end 140.716 92.964) (width 0.1524) (layer F.Cu) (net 20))
 (segment (start 140.716 92.964) (end 140.716 73.152) (width 0.1524) (layer F.Cu) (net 20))
 (segment (start 140.716 73.152) (end 143.764 70.104) (width 0.1524) (layer F.Cu) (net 20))
 (segment (start 143.764 70.104) (end 143.764 69.088) (width 0.1524) (layer F.Cu) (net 20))
 (segment (start 143.51 91.44) (end 146.304 91.44) (width 0.1524) (layer F.Cu) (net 21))
 (segment (start 143.51 86.36) (end 146.304 86.36) (width 0.1524) (layer F.Cu) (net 22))
 (segment (start 143.51 83.82) (end 146.304 83.82) (width 0.1524) (layer F.Cu) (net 23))
 (segment (start 143.51 81.28) (end 146.304 81.28) (width 0.1524) (layer F.Cu) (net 24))
 (segment (start 143.51 78.74) (end 146.304 78.74) (width 0.1524) (layer F.Cu) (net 25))
 (segment (start 146.304 76.2) (end 143.51 76.2) (width 0.1524) (layer F.Cu) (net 26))
 (segment (start 143.51 73.66) (end 146.304 73.66) (width 0.1524) (layer F.Cu) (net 27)))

